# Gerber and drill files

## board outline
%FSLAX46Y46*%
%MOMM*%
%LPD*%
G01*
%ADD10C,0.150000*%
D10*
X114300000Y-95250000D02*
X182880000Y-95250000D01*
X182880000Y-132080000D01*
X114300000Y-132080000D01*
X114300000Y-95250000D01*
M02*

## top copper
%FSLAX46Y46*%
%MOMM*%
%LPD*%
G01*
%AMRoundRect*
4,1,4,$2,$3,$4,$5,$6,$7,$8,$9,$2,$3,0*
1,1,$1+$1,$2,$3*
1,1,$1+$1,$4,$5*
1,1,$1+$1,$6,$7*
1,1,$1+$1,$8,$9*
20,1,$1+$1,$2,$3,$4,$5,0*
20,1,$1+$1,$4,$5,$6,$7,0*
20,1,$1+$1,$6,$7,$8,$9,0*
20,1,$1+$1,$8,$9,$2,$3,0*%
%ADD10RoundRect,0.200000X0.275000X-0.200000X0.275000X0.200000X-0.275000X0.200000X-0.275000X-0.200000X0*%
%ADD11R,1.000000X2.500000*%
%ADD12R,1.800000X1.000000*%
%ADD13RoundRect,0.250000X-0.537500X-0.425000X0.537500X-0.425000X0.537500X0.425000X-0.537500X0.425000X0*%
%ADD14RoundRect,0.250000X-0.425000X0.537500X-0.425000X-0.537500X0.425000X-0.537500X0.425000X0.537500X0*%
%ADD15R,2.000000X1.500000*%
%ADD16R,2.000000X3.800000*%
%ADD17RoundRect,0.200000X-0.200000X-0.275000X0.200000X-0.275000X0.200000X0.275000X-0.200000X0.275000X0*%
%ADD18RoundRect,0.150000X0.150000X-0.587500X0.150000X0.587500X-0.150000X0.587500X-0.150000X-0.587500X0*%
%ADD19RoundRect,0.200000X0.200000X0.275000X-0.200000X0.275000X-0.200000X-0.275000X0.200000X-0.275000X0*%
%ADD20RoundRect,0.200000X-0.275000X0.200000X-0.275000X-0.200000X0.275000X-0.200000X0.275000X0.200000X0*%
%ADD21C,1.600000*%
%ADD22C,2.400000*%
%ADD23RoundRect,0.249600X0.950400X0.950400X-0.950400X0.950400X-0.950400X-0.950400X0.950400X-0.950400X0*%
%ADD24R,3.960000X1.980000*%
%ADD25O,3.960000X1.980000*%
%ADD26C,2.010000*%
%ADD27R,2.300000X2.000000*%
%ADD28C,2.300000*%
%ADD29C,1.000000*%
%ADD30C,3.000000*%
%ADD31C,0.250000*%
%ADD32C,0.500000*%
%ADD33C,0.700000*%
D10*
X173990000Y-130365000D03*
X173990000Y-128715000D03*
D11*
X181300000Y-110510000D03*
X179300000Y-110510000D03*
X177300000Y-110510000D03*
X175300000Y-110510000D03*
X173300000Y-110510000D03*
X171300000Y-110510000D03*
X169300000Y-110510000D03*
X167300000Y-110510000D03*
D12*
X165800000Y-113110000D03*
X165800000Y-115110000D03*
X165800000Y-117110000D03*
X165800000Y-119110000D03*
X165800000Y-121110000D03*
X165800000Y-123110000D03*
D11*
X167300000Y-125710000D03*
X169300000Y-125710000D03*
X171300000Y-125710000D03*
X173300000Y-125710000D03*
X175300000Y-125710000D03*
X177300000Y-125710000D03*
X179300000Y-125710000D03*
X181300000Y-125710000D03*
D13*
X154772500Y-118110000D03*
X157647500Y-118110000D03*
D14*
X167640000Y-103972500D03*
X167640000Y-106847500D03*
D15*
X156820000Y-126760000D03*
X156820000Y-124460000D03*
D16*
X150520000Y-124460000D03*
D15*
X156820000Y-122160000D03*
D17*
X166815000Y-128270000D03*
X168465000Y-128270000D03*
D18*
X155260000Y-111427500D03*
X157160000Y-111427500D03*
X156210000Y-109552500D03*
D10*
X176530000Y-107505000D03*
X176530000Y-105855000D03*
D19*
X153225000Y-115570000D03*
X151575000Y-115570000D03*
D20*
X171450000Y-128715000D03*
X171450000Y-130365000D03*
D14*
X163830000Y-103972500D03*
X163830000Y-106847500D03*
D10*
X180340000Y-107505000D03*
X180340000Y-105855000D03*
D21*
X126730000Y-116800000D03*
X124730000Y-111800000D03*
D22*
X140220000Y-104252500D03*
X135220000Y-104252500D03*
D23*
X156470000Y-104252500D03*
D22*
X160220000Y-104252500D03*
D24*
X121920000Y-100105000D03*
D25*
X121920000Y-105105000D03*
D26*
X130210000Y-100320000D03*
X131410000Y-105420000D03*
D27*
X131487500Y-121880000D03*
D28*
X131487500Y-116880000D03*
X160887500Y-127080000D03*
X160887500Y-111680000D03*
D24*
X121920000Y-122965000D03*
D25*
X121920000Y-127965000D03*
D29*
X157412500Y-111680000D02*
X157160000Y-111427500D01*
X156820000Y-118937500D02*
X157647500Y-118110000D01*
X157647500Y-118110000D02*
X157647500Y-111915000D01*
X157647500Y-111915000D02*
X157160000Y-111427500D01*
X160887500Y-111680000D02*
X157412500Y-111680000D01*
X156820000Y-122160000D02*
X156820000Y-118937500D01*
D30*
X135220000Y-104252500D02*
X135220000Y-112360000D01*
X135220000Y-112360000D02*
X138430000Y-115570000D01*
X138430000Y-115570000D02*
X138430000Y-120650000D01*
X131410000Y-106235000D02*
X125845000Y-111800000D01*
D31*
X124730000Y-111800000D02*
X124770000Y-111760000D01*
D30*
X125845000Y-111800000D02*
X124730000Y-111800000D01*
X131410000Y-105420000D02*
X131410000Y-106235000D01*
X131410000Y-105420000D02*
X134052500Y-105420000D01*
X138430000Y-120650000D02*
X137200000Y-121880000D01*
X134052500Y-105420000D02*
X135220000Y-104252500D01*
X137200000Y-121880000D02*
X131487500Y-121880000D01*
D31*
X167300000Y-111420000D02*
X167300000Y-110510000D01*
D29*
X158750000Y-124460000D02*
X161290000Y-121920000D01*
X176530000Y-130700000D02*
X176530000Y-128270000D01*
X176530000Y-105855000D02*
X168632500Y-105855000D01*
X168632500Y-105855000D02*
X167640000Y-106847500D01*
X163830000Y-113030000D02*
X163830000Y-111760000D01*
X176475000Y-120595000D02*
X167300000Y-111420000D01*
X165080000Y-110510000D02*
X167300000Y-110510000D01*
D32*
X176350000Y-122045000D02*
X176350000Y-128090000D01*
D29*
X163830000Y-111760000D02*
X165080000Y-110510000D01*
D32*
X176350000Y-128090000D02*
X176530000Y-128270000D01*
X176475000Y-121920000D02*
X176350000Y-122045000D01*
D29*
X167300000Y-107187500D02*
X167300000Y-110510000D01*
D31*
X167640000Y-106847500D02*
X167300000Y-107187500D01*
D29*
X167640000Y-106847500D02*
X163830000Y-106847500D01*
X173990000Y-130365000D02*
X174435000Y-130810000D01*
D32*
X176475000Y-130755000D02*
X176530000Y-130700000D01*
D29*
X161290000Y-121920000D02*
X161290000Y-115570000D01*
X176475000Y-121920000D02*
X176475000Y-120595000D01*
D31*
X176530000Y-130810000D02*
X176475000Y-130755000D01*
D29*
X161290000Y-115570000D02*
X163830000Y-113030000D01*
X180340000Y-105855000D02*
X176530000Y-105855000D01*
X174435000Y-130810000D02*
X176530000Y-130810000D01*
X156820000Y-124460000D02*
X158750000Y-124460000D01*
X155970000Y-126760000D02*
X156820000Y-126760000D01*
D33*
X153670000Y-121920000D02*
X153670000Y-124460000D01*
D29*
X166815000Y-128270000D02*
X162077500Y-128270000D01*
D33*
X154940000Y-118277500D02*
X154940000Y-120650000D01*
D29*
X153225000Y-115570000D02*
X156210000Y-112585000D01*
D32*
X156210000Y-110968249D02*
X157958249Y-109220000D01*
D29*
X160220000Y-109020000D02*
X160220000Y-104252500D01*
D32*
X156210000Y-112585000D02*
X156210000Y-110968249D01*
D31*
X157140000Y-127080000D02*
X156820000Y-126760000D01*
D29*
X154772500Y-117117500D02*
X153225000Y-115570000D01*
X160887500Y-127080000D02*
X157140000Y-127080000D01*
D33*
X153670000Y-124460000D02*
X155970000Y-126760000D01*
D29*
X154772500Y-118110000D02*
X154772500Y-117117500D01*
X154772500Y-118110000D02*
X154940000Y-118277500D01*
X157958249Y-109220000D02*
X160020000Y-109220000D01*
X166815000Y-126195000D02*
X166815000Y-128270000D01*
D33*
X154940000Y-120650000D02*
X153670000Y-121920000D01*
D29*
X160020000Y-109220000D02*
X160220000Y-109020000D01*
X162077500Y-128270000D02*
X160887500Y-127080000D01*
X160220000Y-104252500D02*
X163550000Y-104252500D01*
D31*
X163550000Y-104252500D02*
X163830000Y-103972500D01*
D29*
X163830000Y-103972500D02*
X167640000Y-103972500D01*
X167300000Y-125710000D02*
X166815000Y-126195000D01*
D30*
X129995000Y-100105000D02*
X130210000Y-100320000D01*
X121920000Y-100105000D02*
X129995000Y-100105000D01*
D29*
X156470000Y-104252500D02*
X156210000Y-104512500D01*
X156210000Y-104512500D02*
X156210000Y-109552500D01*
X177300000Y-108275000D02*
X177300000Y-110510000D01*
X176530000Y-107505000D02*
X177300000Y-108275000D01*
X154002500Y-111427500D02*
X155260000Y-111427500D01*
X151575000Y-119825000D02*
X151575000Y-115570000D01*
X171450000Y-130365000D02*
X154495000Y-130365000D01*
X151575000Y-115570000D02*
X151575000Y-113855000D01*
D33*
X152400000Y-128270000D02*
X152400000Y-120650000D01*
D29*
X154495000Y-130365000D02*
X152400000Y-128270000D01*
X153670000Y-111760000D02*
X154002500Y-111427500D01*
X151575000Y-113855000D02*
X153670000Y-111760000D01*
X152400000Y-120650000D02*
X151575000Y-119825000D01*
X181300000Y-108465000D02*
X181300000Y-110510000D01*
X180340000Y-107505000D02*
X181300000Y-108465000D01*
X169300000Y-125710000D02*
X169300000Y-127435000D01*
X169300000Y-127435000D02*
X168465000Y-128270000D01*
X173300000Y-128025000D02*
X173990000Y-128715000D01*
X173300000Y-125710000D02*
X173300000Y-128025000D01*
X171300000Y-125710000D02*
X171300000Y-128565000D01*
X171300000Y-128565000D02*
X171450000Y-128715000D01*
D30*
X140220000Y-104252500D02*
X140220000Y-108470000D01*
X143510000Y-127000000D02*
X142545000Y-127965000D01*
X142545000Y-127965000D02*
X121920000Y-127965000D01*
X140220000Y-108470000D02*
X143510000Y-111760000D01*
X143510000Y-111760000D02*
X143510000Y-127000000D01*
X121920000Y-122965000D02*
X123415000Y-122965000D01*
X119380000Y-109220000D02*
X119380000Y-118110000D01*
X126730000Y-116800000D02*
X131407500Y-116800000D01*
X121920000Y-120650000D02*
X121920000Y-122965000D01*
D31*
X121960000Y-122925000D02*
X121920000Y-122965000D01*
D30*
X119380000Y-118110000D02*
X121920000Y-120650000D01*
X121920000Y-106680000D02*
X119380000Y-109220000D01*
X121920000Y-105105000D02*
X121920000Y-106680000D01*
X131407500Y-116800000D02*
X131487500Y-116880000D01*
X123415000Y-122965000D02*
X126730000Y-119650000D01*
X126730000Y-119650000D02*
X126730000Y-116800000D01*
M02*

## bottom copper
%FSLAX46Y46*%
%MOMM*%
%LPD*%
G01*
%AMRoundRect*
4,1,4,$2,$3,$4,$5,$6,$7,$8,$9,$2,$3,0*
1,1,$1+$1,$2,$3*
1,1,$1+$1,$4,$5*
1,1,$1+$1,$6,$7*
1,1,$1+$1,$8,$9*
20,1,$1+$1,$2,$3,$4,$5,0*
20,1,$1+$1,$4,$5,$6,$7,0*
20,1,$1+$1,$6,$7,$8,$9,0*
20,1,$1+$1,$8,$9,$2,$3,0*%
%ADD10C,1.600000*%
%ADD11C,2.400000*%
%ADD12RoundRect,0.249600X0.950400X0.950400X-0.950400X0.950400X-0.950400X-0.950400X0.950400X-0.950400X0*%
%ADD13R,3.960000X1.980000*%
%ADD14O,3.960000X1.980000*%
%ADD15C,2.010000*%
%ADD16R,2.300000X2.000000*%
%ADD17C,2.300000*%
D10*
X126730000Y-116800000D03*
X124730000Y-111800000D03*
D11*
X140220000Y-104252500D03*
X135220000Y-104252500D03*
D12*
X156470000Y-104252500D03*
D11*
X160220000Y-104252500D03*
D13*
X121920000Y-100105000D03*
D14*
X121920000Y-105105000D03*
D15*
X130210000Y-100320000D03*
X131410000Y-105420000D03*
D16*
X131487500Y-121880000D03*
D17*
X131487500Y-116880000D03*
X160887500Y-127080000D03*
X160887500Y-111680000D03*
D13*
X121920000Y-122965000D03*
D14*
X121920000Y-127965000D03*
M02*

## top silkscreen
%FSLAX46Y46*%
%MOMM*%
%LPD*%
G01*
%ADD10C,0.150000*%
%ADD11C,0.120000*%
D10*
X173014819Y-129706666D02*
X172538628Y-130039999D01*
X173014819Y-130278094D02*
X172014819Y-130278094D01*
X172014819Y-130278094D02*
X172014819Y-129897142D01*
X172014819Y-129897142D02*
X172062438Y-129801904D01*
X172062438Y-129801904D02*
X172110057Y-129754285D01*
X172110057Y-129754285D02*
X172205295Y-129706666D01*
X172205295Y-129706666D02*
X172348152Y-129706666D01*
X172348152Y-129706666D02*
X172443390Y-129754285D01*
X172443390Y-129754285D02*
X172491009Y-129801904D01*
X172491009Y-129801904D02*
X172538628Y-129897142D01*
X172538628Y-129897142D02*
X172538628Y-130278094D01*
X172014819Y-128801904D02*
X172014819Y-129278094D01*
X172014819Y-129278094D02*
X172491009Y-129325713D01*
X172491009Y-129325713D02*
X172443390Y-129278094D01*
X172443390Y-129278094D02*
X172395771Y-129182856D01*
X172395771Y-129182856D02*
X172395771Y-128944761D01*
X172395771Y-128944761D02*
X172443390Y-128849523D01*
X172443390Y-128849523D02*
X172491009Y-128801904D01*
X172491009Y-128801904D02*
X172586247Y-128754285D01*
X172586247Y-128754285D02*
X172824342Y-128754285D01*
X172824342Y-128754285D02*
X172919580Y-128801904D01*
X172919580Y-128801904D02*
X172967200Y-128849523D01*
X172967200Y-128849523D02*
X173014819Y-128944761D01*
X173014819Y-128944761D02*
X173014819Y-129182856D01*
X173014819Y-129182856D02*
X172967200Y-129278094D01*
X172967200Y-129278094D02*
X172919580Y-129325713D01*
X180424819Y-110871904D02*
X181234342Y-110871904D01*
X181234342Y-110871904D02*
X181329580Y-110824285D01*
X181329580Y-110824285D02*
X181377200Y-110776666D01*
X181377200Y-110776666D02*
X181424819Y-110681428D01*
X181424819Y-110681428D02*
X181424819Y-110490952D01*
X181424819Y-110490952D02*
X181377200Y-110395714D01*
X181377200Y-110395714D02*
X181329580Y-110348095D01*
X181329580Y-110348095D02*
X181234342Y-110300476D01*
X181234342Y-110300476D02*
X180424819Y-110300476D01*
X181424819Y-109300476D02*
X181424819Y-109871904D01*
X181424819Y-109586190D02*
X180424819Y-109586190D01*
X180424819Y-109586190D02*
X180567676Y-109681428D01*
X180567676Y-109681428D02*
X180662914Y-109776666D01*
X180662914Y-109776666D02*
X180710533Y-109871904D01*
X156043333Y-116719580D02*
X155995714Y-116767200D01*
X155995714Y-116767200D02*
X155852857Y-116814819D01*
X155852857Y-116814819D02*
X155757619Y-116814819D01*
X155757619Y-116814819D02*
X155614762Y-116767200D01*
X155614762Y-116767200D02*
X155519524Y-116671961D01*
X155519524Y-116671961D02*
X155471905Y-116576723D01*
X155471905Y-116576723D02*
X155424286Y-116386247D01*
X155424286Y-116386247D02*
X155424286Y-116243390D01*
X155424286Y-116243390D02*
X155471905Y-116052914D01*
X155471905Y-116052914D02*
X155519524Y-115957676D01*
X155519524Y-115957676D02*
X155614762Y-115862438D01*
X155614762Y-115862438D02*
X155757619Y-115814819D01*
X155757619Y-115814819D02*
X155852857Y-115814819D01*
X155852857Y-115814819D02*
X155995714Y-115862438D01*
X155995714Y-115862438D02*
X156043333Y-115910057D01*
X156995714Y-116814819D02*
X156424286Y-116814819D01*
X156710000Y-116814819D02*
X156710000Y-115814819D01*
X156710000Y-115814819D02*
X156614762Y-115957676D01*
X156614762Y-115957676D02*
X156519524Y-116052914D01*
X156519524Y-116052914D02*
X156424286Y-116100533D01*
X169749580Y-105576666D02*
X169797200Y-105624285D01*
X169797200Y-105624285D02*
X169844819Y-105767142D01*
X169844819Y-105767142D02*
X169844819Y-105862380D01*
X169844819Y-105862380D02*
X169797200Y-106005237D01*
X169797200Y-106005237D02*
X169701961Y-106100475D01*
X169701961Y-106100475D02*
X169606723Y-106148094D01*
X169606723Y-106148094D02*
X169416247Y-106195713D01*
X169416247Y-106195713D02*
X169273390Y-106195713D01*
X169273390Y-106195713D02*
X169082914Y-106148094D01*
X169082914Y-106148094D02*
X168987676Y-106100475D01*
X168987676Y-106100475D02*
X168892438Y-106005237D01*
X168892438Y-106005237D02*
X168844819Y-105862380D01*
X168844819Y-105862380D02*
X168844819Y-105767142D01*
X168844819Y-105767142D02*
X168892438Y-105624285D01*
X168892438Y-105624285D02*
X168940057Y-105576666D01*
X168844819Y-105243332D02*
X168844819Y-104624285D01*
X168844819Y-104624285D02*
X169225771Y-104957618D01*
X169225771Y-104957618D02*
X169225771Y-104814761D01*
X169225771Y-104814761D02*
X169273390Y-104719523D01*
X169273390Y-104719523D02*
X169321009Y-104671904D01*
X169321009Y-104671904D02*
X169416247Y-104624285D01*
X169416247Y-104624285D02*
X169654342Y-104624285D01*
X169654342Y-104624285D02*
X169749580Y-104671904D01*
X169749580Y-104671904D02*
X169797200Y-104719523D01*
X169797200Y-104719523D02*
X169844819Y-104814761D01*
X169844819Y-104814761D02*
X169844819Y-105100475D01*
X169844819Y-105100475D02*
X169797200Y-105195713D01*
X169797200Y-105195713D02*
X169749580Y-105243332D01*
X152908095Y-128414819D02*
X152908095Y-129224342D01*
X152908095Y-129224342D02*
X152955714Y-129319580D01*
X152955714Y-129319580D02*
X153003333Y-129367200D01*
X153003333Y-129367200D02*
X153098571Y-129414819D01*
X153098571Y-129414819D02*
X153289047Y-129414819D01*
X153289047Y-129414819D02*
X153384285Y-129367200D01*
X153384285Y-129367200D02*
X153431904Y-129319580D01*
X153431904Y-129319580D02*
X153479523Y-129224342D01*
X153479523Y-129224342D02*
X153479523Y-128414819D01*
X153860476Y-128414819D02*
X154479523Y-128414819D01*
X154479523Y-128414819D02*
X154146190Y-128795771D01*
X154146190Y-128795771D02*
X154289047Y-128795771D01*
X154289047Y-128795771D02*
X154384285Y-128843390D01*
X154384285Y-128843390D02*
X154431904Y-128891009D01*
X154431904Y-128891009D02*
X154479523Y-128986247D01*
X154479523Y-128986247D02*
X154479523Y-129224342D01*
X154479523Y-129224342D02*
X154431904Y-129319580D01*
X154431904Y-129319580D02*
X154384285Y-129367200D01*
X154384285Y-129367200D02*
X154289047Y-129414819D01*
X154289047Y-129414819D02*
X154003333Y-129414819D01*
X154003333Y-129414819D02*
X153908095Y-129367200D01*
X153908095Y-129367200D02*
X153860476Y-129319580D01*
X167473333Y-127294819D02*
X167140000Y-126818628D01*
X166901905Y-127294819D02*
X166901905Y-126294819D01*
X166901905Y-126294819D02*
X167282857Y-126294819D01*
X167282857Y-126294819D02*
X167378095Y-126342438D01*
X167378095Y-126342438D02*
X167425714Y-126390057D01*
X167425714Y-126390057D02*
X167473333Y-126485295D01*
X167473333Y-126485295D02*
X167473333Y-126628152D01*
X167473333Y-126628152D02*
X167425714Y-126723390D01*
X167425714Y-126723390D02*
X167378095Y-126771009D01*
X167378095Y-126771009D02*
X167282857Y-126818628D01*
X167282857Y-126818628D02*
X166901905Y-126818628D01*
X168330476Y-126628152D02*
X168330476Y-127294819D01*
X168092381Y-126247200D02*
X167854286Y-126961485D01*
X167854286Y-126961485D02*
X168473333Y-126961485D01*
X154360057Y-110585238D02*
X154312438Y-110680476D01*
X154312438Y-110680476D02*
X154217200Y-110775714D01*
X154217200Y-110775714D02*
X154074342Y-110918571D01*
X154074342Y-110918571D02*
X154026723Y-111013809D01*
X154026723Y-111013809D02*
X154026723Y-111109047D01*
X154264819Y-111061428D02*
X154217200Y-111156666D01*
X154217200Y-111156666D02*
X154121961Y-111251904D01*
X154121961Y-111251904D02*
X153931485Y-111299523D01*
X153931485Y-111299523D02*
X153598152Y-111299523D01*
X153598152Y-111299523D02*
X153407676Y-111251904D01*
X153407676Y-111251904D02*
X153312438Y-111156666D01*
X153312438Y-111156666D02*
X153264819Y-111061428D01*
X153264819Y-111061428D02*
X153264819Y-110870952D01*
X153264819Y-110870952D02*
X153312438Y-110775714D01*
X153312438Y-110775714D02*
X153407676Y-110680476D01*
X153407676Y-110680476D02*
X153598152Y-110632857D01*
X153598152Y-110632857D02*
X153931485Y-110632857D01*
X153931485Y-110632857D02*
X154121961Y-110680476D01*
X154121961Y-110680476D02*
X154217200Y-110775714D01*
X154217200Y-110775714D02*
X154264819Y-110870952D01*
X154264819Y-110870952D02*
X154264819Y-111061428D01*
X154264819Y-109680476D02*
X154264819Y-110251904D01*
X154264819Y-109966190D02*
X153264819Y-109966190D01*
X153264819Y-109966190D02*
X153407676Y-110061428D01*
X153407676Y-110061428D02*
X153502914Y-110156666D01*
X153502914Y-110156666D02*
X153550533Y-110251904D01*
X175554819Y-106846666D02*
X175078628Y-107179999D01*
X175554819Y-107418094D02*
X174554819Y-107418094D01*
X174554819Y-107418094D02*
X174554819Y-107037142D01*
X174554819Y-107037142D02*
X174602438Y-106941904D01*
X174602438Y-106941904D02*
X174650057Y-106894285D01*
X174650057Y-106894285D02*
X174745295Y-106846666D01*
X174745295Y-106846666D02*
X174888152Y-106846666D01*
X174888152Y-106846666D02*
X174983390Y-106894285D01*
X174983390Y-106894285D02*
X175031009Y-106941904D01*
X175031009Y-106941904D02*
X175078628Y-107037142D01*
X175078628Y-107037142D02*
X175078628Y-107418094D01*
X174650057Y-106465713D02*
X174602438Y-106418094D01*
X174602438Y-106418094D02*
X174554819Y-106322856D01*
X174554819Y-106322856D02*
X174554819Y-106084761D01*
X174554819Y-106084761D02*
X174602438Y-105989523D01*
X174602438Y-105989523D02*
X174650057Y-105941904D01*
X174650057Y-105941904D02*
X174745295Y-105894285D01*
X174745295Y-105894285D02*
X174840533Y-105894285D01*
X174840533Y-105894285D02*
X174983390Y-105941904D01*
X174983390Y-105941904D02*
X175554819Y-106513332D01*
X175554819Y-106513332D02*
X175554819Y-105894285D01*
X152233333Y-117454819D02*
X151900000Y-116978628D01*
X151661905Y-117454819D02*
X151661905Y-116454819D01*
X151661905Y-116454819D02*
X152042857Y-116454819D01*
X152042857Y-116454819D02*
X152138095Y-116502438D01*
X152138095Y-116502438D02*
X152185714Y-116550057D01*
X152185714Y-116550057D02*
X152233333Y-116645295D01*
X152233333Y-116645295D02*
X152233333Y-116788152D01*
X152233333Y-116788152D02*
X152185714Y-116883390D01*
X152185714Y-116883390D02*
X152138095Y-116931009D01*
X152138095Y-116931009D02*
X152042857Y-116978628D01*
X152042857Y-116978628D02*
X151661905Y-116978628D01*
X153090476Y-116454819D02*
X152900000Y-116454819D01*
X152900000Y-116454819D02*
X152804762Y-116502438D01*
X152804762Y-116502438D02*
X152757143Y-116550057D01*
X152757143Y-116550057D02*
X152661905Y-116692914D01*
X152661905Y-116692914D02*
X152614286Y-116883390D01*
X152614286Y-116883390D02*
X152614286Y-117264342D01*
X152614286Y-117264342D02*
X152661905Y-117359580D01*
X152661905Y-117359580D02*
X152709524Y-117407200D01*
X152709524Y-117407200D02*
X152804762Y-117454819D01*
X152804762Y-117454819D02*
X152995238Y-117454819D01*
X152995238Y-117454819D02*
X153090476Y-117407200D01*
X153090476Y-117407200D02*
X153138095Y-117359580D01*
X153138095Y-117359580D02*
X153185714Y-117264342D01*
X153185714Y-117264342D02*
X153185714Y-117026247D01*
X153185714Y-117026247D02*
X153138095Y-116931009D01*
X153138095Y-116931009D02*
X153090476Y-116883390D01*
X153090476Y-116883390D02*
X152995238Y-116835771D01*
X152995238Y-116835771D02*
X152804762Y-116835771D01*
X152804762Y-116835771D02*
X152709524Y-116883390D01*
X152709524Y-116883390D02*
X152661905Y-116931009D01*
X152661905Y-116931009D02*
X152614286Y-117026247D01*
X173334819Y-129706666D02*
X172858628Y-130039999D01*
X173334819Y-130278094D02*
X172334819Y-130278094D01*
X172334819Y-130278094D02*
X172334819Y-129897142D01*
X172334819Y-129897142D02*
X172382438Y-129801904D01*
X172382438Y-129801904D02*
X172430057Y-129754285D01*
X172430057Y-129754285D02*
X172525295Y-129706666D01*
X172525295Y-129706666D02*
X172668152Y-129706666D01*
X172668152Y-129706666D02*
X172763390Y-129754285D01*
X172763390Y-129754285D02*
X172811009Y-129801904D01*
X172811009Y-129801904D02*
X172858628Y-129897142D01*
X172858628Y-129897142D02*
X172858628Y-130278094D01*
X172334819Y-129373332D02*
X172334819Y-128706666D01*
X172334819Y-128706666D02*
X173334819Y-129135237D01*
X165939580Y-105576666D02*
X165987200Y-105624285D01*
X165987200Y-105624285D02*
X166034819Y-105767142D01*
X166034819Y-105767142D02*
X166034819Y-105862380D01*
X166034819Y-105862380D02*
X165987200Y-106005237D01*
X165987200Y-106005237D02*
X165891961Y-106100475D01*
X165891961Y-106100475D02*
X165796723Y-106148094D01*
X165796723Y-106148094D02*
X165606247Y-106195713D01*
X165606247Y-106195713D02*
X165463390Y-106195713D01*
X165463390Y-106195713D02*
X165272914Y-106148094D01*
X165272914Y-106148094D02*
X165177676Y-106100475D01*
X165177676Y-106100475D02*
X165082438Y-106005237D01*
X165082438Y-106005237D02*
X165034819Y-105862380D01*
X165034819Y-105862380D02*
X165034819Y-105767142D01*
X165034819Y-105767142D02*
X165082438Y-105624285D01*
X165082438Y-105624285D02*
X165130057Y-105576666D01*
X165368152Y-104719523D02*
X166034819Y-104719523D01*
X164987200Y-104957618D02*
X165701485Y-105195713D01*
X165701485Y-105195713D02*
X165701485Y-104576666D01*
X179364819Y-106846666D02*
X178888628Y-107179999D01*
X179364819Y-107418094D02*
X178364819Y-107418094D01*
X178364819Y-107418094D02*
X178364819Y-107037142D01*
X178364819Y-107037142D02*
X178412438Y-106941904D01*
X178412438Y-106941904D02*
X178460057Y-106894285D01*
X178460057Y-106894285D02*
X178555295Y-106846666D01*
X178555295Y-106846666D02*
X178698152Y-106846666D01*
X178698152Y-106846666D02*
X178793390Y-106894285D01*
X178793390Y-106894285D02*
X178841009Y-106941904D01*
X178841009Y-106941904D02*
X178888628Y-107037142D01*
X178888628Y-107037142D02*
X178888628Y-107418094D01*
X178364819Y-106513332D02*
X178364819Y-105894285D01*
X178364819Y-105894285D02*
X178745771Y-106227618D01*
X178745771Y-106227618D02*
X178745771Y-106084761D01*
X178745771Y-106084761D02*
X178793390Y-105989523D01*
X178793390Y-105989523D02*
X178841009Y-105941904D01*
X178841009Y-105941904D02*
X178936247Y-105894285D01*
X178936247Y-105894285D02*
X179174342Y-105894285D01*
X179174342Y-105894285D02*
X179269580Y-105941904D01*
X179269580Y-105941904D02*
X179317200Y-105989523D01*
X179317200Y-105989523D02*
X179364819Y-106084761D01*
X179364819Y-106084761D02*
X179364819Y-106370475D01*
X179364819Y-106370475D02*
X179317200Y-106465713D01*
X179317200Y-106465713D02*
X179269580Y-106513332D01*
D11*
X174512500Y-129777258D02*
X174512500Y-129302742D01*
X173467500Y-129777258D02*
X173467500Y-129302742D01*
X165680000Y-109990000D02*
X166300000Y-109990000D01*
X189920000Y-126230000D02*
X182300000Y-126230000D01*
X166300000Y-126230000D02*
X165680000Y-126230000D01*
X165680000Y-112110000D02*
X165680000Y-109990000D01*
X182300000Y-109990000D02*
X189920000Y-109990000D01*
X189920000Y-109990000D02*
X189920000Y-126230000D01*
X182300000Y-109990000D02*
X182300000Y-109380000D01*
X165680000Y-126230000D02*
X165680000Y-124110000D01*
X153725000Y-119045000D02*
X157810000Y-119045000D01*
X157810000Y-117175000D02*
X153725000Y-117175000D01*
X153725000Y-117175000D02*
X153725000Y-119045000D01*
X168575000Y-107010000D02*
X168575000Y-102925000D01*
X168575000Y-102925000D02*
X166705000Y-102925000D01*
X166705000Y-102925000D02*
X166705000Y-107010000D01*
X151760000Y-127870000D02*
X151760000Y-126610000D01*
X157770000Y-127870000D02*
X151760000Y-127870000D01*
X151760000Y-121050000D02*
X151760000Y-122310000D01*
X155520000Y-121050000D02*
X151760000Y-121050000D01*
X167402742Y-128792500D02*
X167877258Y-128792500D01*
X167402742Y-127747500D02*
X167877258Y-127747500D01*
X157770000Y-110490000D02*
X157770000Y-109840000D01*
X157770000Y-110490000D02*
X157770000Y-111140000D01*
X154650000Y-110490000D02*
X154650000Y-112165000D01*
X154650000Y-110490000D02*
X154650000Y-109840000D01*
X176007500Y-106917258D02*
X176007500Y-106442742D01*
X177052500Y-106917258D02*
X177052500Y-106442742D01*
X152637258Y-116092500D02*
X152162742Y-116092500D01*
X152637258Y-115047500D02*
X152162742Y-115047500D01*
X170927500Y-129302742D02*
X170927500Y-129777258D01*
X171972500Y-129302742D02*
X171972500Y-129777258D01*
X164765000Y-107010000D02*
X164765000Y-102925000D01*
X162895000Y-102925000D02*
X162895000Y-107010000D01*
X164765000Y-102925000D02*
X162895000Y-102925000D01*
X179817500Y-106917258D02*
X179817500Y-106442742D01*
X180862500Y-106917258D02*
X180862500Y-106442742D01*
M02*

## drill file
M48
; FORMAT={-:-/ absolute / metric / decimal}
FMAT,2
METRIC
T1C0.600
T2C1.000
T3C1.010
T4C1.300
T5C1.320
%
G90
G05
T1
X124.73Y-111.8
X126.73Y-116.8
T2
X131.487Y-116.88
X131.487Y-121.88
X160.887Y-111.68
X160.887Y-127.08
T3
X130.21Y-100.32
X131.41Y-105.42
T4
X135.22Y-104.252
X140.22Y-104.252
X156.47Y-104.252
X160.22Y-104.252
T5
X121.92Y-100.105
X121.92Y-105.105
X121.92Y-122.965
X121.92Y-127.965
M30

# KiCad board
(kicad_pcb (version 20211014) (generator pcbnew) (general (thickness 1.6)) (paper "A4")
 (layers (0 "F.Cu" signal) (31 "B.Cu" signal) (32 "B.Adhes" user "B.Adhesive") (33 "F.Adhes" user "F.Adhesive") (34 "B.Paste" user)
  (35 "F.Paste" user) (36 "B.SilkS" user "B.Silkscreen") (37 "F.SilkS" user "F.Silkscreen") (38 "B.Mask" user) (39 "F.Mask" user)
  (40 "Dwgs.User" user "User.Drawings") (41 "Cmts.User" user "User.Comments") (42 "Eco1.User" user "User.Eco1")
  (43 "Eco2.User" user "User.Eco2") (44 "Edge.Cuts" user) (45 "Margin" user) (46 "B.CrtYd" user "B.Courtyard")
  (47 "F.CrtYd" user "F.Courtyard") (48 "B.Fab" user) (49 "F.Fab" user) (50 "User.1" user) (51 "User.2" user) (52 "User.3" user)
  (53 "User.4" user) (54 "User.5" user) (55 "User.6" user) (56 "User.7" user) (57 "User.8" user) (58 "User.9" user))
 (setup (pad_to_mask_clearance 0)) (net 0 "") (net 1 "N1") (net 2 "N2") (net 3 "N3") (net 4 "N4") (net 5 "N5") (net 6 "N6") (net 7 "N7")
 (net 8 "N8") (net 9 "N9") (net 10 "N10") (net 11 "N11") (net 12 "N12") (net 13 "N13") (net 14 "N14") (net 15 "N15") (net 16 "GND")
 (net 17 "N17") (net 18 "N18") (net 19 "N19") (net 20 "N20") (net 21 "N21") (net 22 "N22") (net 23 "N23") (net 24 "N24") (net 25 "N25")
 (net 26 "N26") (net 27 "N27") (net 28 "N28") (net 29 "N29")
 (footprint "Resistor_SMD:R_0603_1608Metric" (layer "F.Cu") (at 173.99 129.54 90)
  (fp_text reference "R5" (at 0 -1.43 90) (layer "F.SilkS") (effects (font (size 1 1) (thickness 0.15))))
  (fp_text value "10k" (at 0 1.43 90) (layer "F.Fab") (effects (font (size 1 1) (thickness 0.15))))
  (fp_line (start -0.237258 0.5225) (end 0.237258 0.5225) (layer "F.SilkS") (width 0.12))
  (fp_line (start -0.237258 -0.5225) (end 0.237258 -0.5225) (layer "F.SilkS") (width 0.12))
  (pad "1" smd roundrect (at -0.825 0 90) (size 0.8 0.95) (layers "F.Cu" "F.Paste" "F.Mask") (roundrect_rratio 0.25) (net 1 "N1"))
  (pad "2" smd roundrect (at 0.825 0 90) (size 0.8 0.95) (layers "F.Cu" "F.Paste" "F.Mask") (roundrect_rratio 0.25) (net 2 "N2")))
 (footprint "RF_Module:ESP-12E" (layer "F.Cu") (at 177.8 118.11 -90)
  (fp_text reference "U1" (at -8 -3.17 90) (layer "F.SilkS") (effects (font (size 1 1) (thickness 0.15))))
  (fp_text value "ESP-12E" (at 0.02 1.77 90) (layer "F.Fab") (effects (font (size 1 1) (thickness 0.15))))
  (fp_line (start -8.12 12.12) (end -8.12 11.5) (layer "F.SilkS") (width 0.12))
  (fp_line (start 8.12 -12.12) (end 8.12 -4.5) (layer "F.SilkS") (width 0.12))
  (fp_line (start 8.12 11.5) (end 8.12 12.12) (layer "F.SilkS") (width 0.12))
  (fp_line (start -6 12.12) (end -8.12 12.12) (layer "F.SilkS") (width 0.12))
  (fp_line (start -8.12 -4.5) (end -8.12 -12.12) (layer "F.SilkS") (width 0.12))
  (fp_line (start -8.12 -12.12) (end 8.12 -12.12) (layer "F.SilkS") (width 0.12))
  (fp_line (start -8.12 -4.5) (end -8.73 -4.5) (layer "F.SilkS") (width 0.12))
  (fp_line (start 8.12 12.12) (end 6 12.12) (layer "F.SilkS") (width 0.12))
  (pad "1" smd rect (at -7.6 -3.5 270) (size 2.5 1) (layers "F.Cu" "F.Paste" "F.Mask") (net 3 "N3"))
  (pad "2" smd rect (at -7.6 -1.5 270) (size 2.5 1) (layers "F.Cu" "F.Paste" "F.Mask") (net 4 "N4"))
  (pad "3" smd rect (at -7.6 0.5 270) (size 2.5 1) (layers "F.Cu" "F.Paste" "F.Mask") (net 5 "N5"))
  (pad "4" smd rect (at -7.6 2.5 270) (size 2.5 1) (layers "F.Cu" "F.Paste" "F.Mask") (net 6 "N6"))
  (pad "5" smd rect (at -7.6 4.5 270) (size 2.5 1) (layers "F.Cu" "F.Paste" "F.Mask") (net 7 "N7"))
  (pad "6" smd rect (at -7.6 6.5 270) (size 2.5 1) (layers "F.Cu" "F.Paste" "F.Mask") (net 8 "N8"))
  (pad "7" smd rect (at -7.6 8.5 270) (size 2.5 1) (layers "F.Cu" "F.Paste" "F.Mask") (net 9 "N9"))
  (pad "8" smd rect (at -7.6 10.5 270) (size 2.5 1) (layers "F.Cu" "F.Paste" "F.Mask") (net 1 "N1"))
  (pad "9" smd rect (at -5 12 270) (size 1 1.8) (layers "F.Cu" "F.Paste" "F.Mask") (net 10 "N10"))
  (pad "10" smd rect (at -3 12 270) (size 1 1.8) (layers "F.Cu" "F.Paste" "F.Mask") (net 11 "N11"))
  (pad "11" smd rect (at -1 12 270) (size 1 1.8) (layers "F.Cu" "F.Paste" "F.Mask") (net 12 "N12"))
  (pad "12" smd rect (at 1 12 270) (size 1 1.8) (layers "F.Cu" "F.Paste" "F.Mask") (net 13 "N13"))
  (pad "13" smd rect (at 3 12 270) (size 1 1.8) (layers "F.Cu" "F.Paste" "F.Mask") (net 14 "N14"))
  (pad "14" smd rect (at 5 12 270) (size 1 1.8) (layers "F.Cu" "F.Paste" "F.Mask") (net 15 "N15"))
  (pad "15" smd rect (at 7.6 10.5 270) (size 2.5 1) (layers "F.Cu" "F.Paste" "F.Mask") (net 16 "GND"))
  (pad "16" smd rect (at 7.6 8.5 270) (size 2.5 1) (layers "F.Cu" "F.Paste" "F.Mask") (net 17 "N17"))
  (pad "17" smd rect (at 7.6 6.5 270) (size 2.5 1) (layers "F.Cu" "F.Paste" "F.Mask") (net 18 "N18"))
  (pad "18" smd rect (at 7.6 4.5 270) (size 2.5 1) (layers "F.Cu" "F.Paste" "F.Mask") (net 2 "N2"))
  (pad "19" smd rect (at 7.6 2.5 270) (size 2.5 1) (layers "F.Cu" "F.Paste" "F.Mask") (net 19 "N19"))
  (pad "20" smd rect (at 7.6 0.5 270) (size 2.5 1) (layers "F.Cu" "F.Paste" "F.Mask") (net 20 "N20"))
  (pad "21" smd rect (at 7.6 -1.5 270) (size 2.5 1) (layers "F.Cu" "F.Paste" "F.Mask") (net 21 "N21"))
  (pad "22" smd rect (at 7.6 -3.5 270) (size 2.5 1) (layers "F.Cu" "F.Paste" "F.Mask") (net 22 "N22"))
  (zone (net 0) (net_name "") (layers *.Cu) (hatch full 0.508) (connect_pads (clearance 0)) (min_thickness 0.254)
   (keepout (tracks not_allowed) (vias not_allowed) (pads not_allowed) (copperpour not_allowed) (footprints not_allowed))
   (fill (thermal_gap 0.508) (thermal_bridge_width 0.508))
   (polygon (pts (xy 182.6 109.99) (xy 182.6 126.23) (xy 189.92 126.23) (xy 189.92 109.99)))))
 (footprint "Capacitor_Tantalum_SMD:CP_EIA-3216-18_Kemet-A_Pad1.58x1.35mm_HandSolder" (layer "F.Cu") (at 156.21 118.11)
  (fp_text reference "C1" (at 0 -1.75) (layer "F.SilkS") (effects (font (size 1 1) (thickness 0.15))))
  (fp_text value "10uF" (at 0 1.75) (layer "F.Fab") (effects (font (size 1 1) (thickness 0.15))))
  (fp_line (start -2.485 0.935) (end 1.6 0.935) (layer "F.SilkS") (width 0.12))
  (fp_line (start 1.6 -0.935) (end -2.485 -0.935) (layer "F.SilkS") (width 0.12))
  (fp_line (start -2.485 -0.935) (end -2.485 0.935) (layer "F.SilkS") (width 0.12))
  (pad "1" smd roundrect (at -1.4375 0) (size 1.575 1.35) (layers "F.Cu" "F.Paste" "F.Mask") (roundrect_rratio 0.1851851852) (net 16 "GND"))
  (pad "2" smd roundrect (at 1.4375 0) (size 1.575 1.35) (layers "F.Cu" "F.Paste" "F.Mask") (roundrect_rratio 0.1851851852) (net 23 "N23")))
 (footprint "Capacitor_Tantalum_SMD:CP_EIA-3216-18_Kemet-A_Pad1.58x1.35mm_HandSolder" (layer "F.Cu") (at 167.64 105.41 -90)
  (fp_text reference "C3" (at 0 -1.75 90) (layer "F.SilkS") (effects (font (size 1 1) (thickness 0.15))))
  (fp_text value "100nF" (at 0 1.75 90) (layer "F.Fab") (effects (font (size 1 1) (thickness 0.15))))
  (fp_line (start 1.6 -0.935) (end -2.485 -0.935) (layer "F.SilkS") (width 0.12))
  (fp_line (start -2.485 -0.935) (end -2.485 0.935) (layer "F.SilkS") (width 0.12))
  (fp_line (start -2.485 0.935) (end 1.6 0.935) (layer "F.SilkS") (width 0.12))
  (pad "1" smd roundrect (at -1.4375 0 270) (size 1.575 1.35) (layers "F.Cu" "F.Paste" "F.Mask") (roundrect_rratio 0.1851851852)
   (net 16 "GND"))
  (pad "2" smd roundrect (at 1.4375 0 270) (size 1.575 1.35) (layers "F.Cu" "F.Paste" "F.Mask") (roundrect_rratio 0.1851851852) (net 1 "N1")))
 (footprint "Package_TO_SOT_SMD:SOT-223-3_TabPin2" (layer "F.Cu") (at 153.67 124.46 180)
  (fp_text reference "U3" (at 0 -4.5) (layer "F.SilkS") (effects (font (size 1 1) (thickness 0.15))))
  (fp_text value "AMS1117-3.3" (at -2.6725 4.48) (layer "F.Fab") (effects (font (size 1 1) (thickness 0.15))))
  (fp_line (start 1.91 -3.41) (end 1.91 -2.15) (layer "F.SilkS") (width 0.12))
  (fp_line (start -4.1 -3.41) (end 1.91 -3.41) (layer "F.SilkS") (width 0.12))
  (fp_line (start 1.91 3.41) (end 1.91 2.15) (layer "F.SilkS") (width 0.12))
  (fp_line (start -1.85 3.41) (end 1.91 3.41) (layer "F.SilkS") (width 0.12))
  (pad "1" smd rect (at -3.15 -2.3 180) (size 2 1.5) (layers "F.Cu" "F.Paste" "F.Mask") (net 16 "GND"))
  (pad "2" smd rect (at -3.15 0 180) (size 2 1.5) (layers "F.Cu" "F.Paste" "F.Mask") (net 1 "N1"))
  (pad "2" smd rect (at 3.15 0 180) (size 2 3.8) (layers "F.Cu" "F.Paste" "F.Mask") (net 1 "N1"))
  (pad "3" smd rect (at -3.15 2.3 180) (size 2 1.5) (layers "F.Cu" "F.Paste" "F.Mask") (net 23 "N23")))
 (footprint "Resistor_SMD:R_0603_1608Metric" (layer "F.Cu") (at 167.64 128.27)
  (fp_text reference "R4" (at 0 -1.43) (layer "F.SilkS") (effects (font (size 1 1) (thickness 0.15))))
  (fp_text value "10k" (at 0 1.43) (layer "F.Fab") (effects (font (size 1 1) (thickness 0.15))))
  (fp_line (start -0.237258 0.5225) (end 0.237258 0.5225) (layer "F.SilkS") (width 0.12))
  (fp_line (start -0.237258 -0.5225) (end 0.237258 -0.5225) (layer "F.SilkS") (width 0.12))
  (pad "1" smd roundrect (at -0.825 0) (size 0.8 0.95) (layers "F.Cu" "F.Paste" "F.Mask") (roundrect_rratio 0.25) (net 16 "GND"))
  (pad "2" smd roundrect (at 0.825 0) (size 0.8 0.95) (layers "F.Cu" "F.Paste" "F.Mask") (roundrect_rratio 0.25) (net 17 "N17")))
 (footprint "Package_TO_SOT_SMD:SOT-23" (layer "F.Cu") (at 156.21 110.49 90)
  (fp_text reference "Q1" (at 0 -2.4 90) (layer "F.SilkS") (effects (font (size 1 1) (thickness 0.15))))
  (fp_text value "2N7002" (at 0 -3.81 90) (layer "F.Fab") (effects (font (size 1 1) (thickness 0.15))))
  (fp_line (start 0 1.56) (end 0.65 1.56) (layer "F.SilkS") (width 0.12))
  (fp_line (start 0 1.56) (end -0.65 1.56) (layer "F.SilkS") (width 0.12))
  (fp_line (start 0 -1.56) (end -1.675 -1.56) (layer "F.SilkS") (width 0.12))
  (fp_line (start 0 -1.56) (end 0.65 -1.56) (layer "F.SilkS") (width 0.12))
  (pad "1" smd roundrect (at -0.9375 -0.95 90) (size 1.475 0.6) (layers "F.Cu" "F.Paste" "F.Mask") (roundrect_rratio 0.25) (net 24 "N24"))
  (pad "2" smd roundrect (at -0.9375 0.95 90) (size 1.475 0.6) (layers "F.Cu" "F.Paste" "F.Mask") (roundrect_rratio 0.25) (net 23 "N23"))
  (pad "3" smd roundrect (at 0.9375 0 90) (size 1.475 0.6) (layers "F.Cu" "F.Paste" "F.Mask") (roundrect_rratio 0.25) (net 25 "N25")))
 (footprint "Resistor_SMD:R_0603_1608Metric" (layer "F.Cu") (at 176.53 106.68 90)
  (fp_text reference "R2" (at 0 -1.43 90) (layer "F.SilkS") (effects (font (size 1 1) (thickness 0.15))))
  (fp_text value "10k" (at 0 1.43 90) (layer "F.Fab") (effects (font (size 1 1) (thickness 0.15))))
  (fp_line (start -0.237258 -0.5225) (end 0.237258 -0.5225) (layer "F.SilkS") (width 0.12))
  (fp_line (start -0.237258 0.5225) (end 0.237258 0.5225) (layer "F.SilkS") (width 0.12))
  (pad "1" smd roundrect (at -0.825 0 90) (size 0.8 0.95) (layers "F.Cu" "F.Paste" "F.Mask") (roundrect_rratio 0.25) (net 5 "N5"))
  (pad "2" smd roundrect (at 0.825 0 90) (size 0.8 0.95) (layers "F.Cu" "F.Paste" "F.Mask") (roundrect_rratio 0.25) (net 1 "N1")))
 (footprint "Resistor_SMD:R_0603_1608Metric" (layer "F.Cu") (at 152.4 115.57 180)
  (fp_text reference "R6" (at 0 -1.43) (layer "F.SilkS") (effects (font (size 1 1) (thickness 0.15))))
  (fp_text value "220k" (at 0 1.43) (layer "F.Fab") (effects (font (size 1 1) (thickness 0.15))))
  (fp_line (start -0.237258 -0.5225) (end 0.237258 -0.5225) (layer "F.SilkS") (width 0.12))
  (fp_line (start -0.237258 0.5225) (end 0.237258 0.5225) (layer "F.SilkS") (width 0.12))
  (pad "1" smd roundrect (at -0.825 0 180) (size 0.8 0.95) (layers "F.Cu" "F.Paste" "F.Mask") (roundrect_rratio 0.25) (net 16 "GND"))
  (pad "2" smd roundrect (at 0.825 0 180) (size 0.8 0.95) (layers "F.Cu" "F.Paste" "F.Mask") (roundrect_rratio 0.25) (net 24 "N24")))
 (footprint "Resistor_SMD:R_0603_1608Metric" (layer "F.Cu") (at 171.45 129.54 -90)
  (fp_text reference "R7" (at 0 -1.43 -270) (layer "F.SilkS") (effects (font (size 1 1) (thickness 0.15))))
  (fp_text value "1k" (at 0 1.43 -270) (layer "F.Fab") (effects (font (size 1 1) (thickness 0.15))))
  (fp_line (start -0.237258 0.5225) (end 0.237258 0.5225) (layer "F.SilkS") (width 0.12))
  (fp_line (start -0.237258 -0.5225) (end 0.237258 -0.5225) (layer "F.SilkS") (width 0.12))
  (pad "1" smd roundrect (at -0.825 0 270) (size 0.8 0.95) (layers "F.Cu" "F.Paste" "F.Mask") (roundrect_rratio 0.25) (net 18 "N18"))
  (pad "2" smd roundrect (at 0.825 0 270) (size 0.8 0.95) (layers "F.Cu" "F.Paste" "F.Mask") (roundrect_rratio 0.25) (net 24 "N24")))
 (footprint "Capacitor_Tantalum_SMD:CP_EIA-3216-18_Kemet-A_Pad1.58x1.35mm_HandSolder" (layer "F.Cu") (at 163.83 105.41 -90)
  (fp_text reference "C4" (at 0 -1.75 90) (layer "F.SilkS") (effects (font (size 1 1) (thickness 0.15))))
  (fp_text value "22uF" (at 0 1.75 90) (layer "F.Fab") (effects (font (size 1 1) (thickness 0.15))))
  (fp_line (start 1.6 -0.935) (end -2.485 -0.935) (layer "F.SilkS") (width 0.12))
  (fp_line (start -2.485 0.935) (end 1.6 0.935) (layer "F.SilkS") (width 0.12))
  (fp_line (start -2.485 -0.935) (end -2.485 0.935) (layer "F.SilkS") (width 0.12))
  (pad "1" smd roundrect (at -1.4375 0 270) (size 1.575 1.35) (layers "F.Cu" "F.Paste" "F.Mask") (roundrect_rratio 0.1851851852)
   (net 16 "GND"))
  (pad "2" smd roundrect (at 1.4375 0 270) (size 1.575 1.35) (layers "F.Cu" "F.Paste" "F.Mask") (roundrect_rratio 0.1851851852) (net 1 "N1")))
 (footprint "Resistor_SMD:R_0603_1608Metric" (layer "F.Cu") (at 180.34 106.68 90)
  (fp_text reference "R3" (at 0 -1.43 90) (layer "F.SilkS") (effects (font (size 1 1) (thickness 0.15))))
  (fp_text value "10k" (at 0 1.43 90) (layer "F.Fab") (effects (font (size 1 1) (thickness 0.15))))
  (fp_line (start -0.237258 -0.5225) (end 0.237258 -0.5225) (layer "F.SilkS") (width 0.12))
  (fp_line (start -0.237258 0.5225) (end 0.237258 0.5225) (layer "F.SilkS") (width 0.12))
  (pad "1" smd roundrect (at -0.825 0 90) (size 0.8 0.95) (layers "F.Cu" "F.Paste" "F.Mask") (roundrect_rratio 0.25) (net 3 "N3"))
  (pad "2" smd roundrect (at 0.825 0 90) (size 0.8 0.95) (layers "F.Cu" "F.Paste" "F.Mask") (roundrect_rratio 0.25) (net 1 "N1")))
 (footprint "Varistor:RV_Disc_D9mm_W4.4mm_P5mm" (layer "B.Cu") (at 126.73 116.8 90)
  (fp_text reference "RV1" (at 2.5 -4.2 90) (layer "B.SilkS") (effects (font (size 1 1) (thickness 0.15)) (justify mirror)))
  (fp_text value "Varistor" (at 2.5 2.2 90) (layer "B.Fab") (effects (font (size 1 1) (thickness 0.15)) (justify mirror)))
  (pad "1" thru_hole circle (at 0 0 90) (size 1.6 1.6) (drill 0.6) (layers *.Cu *.Mask) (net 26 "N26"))
  (pad "2" thru_hole circle (at 5 -2 90) (size 1.6 1.6) (drill 0.6) (layers *.Cu *.Mask) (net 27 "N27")))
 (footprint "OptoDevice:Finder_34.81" (layer "B.Cu") (at 156.47 104.2525 180)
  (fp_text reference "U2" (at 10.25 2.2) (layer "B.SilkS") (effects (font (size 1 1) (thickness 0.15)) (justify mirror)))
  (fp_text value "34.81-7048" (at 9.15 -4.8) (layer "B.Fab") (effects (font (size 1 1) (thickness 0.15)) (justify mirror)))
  (pad "11" thru_hole circle (at 16.25 0 180) (size 2.4 2.4) (drill 1.3) (layers *.Cu *.Mask) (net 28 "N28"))
  (pad "14" thru_hole circle (at 21.25 0 180) (size 2.4 2.4) (drill 1.3) (layers *.Cu *.Mask) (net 27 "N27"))
  (pad "A1" thru_hole roundrect (at 0 0 180) (size 2.4 2.4) (drill 1.3) (layers *.Cu *.Mask) (roundrect_rratio 0.104) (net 25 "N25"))
  (pad "A2" thru_hole circle (at -3.75 0 180) (size 2.4 2.4) (drill 1.3) (layers *.Cu *.Mask) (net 16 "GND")))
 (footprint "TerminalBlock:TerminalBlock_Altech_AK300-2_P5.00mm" (layer "B.Cu") (at 121.92 100.105 -90)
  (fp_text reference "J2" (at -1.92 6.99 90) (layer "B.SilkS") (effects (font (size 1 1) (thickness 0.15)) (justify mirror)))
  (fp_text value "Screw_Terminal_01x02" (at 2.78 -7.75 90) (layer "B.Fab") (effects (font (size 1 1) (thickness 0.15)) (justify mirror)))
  (pad "1" thru_hole rect (at 0 0 270) (size 1.98 3.96) (drill 1.32) (layers *.Cu *.Mask) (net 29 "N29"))
  (pad "2" thru_hole oval (at 5 0 270) (size 1.98 3.96) (drill 1.32) (layers *.Cu *.Mask) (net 26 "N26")))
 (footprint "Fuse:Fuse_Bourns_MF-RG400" (layer "B.Cu") (at 130.21 100.32 -90)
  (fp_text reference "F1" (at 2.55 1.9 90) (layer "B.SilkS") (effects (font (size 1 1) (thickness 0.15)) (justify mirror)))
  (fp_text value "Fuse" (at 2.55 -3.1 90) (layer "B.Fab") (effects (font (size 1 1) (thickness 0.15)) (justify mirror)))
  (pad "1" thru_hole circle (at 0 0 270) (size 2.01 2.01) (drill 1.01) (layers *.Cu *.Mask) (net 29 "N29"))
  (pad "2" thru_hole circle (at 5.1 -1.2 270) (size 2.01 2.01) (drill 1.01) (layers *.Cu *.Mask) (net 27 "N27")))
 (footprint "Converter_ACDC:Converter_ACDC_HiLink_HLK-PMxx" (layer "B.Cu") (at 131.4875 121.88)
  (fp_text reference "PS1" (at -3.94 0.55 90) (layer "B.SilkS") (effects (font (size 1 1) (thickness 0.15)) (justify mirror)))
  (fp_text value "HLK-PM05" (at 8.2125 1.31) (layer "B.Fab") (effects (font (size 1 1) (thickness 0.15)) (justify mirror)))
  (pad "1" thru_hole rect (at 0 0) (size 2.3 2) (drill 1) (layers *.Cu *.Mask) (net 27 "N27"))
  (pad "2" thru_hole circle (at 0 -5) (size 2.3 2.3) (drill 1) (layers *.Cu *.Mask) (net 26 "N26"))
  (pad "3" thru_hole circle (at 29.4 5.2) (size 2.3 2.3) (drill 1) (layers *.Cu *.Mask) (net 16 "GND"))
  (pad "4" thru_hole circle (at 29.4 -10.2) (size 2.3 2.3) (drill 1) (layers *.Cu *.Mask) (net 23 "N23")))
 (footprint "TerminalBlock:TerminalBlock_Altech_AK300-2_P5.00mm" (layer "B.Cu") (at 121.92 122.965 -90)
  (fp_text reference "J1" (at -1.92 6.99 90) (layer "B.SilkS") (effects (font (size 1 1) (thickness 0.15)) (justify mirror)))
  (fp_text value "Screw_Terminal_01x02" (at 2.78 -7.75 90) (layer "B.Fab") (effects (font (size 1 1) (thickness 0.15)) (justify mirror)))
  (pad "1" thru_hole rect (at 0 0 270) (size 1.98 3.96) (drill 1.32) (layers *.Cu *.Mask) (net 26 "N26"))
  (pad "2" thru_hole oval (at 5 0 270) (size 1.98 3.96) (drill 1.32) (layers *.Cu *.Mask) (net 28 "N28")))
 (gr_rect (start 114.3 95.25) (end 182.88 132.08) (layer "Edge.Cuts") (width 0.15) (fill none))
 (segment (start 157.4125 111.68) (end 157.16 111.4275) (width 1) (layer "F.Cu") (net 23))
 (segment (start 156.82 118.9375) (end 157.6475 118.11) (width 1) (layer "F.Cu") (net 23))
 (segment (start 157.6475 118.11) (end 157.6475 111.915) (width 1) (layer "F.Cu") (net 23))
 (segment (start 157.6475 111.915) (end 157.16 111.4275) (width 1) (layer "F.Cu") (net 23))
 (segment (start 160.8875 111.68) (end 157.4125 111.68) (width 1) (layer "F.Cu") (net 23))
 (segment (start 156.82 122.16) (end 156.82 118.9375) (width 1) (layer "F.Cu") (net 23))
 (segment (start 135.22 104.2525) (end 135.22 112.36) (width 3) (layer "F.Cu") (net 27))
 (segment (start 135.22 112.36) (end 138.43 115.57) (width 3) (layer "F.Cu") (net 27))
 (segment (start 138.43 115.57) (end 138.43 120.65) (width 3) (layer "F.Cu") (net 27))
 (segment (start 131.41 106.235) (end 125.845 111.8) (width 3) (layer "F.Cu") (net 27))
 (segment (start 124.73 111.8) (end 124.77 111.76) (width 0.25) (layer "F.Cu") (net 27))
 (segment (start 125.845 111.8) (end 124.73 111.8) (width 3) (layer "F.Cu") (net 27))
 (segment (start 131.41 105.42) (end 131.41 106.235) (width 3) (layer "F.Cu") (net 27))
 (segment (start 131.41 105.42) (end 134.0525 105.42) (width 3) (layer "F.Cu") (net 27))
 (segment (start 138.43 120.65) (end 137.2 121.88) (width 3) (layer "F.Cu") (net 27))
 (segment (start 134.0525 105.42) (end 135.22 104.2525) (width 3) (layer "F.Cu") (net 27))
 (segment (start 137.2 121.88) (end 131.4875 121.88) (width 3) (layer "F.Cu") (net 27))
 (segment (start 167.3 111.42) (end 167.3 110.51) (width 0.25) (layer "F.Cu") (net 1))
 (segment (start 158.75 124.46) (end 161.29 121.92) (width 1) (layer "F.Cu") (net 1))
 (segment (start 176.53 130.7) (end 176.53 128.27) (width 1) (layer "F.Cu") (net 1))
 (segment (start 176.53 105.855) (end 168.6325 105.855) (width 1) (layer "F.Cu") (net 1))
 (segment (start 168.6325 105.855) (end 167.64 106.8475) (width 1) (layer "F.Cu") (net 1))
 (segment (start 163.83 113.03) (end 163.83 111.76) (width 1) (layer "F.Cu") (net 1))
 (segment (start 176.475 120.595) (end 167.3 111.42) (width 1) (layer "F.Cu") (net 1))
 (segment (start 165.08 110.51) (end 167.3 110.51) (width 1) (layer "F.Cu") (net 1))
 (segment (start 176.35 122.045) (end 176.35 128.09) (width 0.5) (layer "F.Cu") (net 1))
 (segment (start 163.83 111.76) (end 165.08 110.51) (width 1) (layer "F.Cu") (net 1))
 (segment (start 176.35 128.09) (end 176.53 128.27) (width 0.5) (layer "F.Cu") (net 1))
 (segment (start 176.475 121.92) (end 176.35 122.045) (width 0.5) (layer "F.Cu") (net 1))
 (segment (start 167.3 107.1875) (end 167.3 110.51) (width 1) (layer "F.Cu") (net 1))
 (segment (start 167.64 106.8475) (end 167.3 107.1875) (width 0.25) (layer "F.Cu") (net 1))
 (segment (start 167.64 106.8475) (end 163.83 106.8475) (width 1) (layer "F.Cu") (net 1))
 (segment (start 173.99 130.365) (end 174.435 130.81) (width 1) (layer "F.Cu") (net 1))
 (segment (start 176.475 130.755) (end 176.53 130.7) (width 0.5) (layer "F.Cu") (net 1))
 (segment (start 161.29 121.92) (end 161.29 115.57) (width 1) (layer "F.Cu") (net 1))
 (segment (start 176.475 121.92) (end 176.475 120.595) (width 1) (layer "F.Cu") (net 1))
 (segment (start 176.53 130.81) (end 176.475 130.755) (width 0.25) (layer "F.Cu") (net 1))
 (segment (start 161.29 115.57) (end 163.83 113.03) (width 1) (layer "F.Cu") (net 1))
 (segment (start 180.34 105.855) (end 176.53 105.855) (width 1) (layer "F.Cu") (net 1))
 (segment (start 174.435 130.81) (end 176.53 130.81) (width 1) (layer "F.Cu") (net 1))
 (segment (start 156.82 124.46) (end 158.75 124.46) (width 1) (layer "F.Cu") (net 1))
 (segment (start 155.97 126.76) (end 156.82 126.76) (width 1) (layer "F.Cu") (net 16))
 (segment (start 153.67 121.92) (end 153.67 124.46) (width 0.7) (layer "F.Cu") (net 16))
 (segment (start 166.815 128.27) (end 162.0775 128.27) (width 1) (layer "F.Cu") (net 16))
 (segment (start 154.94 118.2775) (end 154.94 120.65) (width 0.7) (layer "F.Cu") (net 16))
 (segment (start 153.225 115.57) (end 156.21 112.585) (width 1) (layer "F.Cu") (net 16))
 (segment (start 156.21 110.968249) (end 157.958249 109.22) (width 0.5) (layer "F.Cu") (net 16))
 (segment (start 160.22 109.02) (end 160.22 104.2525) (width 1) (layer "F.Cu") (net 16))
 (segment (start 156.21 112.585) (end 156.21 110.968249) (width 0.5) (layer "F.Cu") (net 16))
 (segment (start 157.14 127.08) (end 156.82 126.76) (width 0.25) (layer "F.Cu") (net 16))
 (segment (start 154.7725 117.1175) (end 153.225 115.57) (width 1) (layer "F.Cu") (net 16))
 (segment (start 160.8875 127.08) (end 157.14 127.08) (width 1) (layer "F.Cu") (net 16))
 (segment (start 153.67 124.46) (end 155.97 126.76) (width 0.7) (layer "F.Cu") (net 16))
 (segment (start 154.7725 118.11) (end 154.7725 117.1175) (width 1) (layer "F.Cu") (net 16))
 (segment (start 154.7725 118.11) (end 154.94 118.2775) (width 1) (layer "F.Cu") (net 16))
 (segment (start 157.958249 109.22) (end 160.02 109.22) (width 1) (layer "F.Cu") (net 16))
 (segment (start 166.815 126.195) (end 166.815 128.27) (width 1) (layer "F.Cu") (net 16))
 (segment (start 154.94 120.65) (end 153.67 121.92) (width 0.7) (layer "F.Cu") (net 16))
 (segment (start 160.02 109.22) (end 160.22 109.02) (width 1) (layer "F.Cu") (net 16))
 (segment (start 162.0775 128.27) (end 160.8875 127.08) (width 1) (layer "F.Cu") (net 16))
 (segment (start 160.22 104.2525) (end 163.55 104.2525) (width 1) (layer "F.Cu") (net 16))
 (segment (start 163.55 104.2525) (end 163.83 103.9725) (width 0.25) (layer "F.Cu") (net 16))
 (segment (start 163.83 103.9725) (end 167.64 103.9725) (width 1) (layer "F.Cu") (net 16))
 (segment (start 167.3 125.71) (end 166.815 126.195) (width 1) (layer "F.Cu") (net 16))
 (segment (start 129.995 100.105) (end 130.21 100.32) (width 3) (layer "F.Cu") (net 29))
 (segment (start 121.92 100.105) (end 129.995 100.105) (width 3) (layer "F.Cu") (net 29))
 (segment (start 156.47 104.2525) (end 156.21 104.5125) (width 1) (layer "F.Cu") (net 25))
 (segment (start 156.21 104.5125) (end 156.21 109.5525) (width 1) (layer "F.Cu") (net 25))
 (segment (start 177.3 108.275) (end 177.3 110.51) (width 1) (layer "F.Cu") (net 5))
 (segment (start 176.53 107.505) (end 177.3 108.275) (width 1) (layer "F.Cu") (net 5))
 (segment (start 154.0025 111.4275) (end 155.26 111.4275) (width 1) (layer "F.Cu") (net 24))
 (segment (start 151.575 119.825) (end 151.575 115.57) (width 1) (layer "F.Cu") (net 24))
 (segment (start 171.45 130.365) (end 154.495 130.365) (width 1) (layer "F.Cu") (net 24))
 (segment (start 151.575 115.57) (end 151.575 113.855) (width 1) (layer "F.Cu") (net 24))
 (segment (start 152.4 128.27) (end 152.4 120.65) (width 0.7) (layer "F.Cu") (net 24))
 (segment (start 154.495 130.365) (end 152.4 128.27) (width 1) (layer "F.Cu") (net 24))
 (segment (start 153.67 111.76) (end 154.0025 111.4275) (width 1) (layer "F.Cu") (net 24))
 (segment (start 151.575 113.855) (end 153.67 111.76) (width 1) (layer "F.Cu") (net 24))
 (segment (start 152.4 120.65) (end 151.575 119.825) (width 1) (layer "F.Cu") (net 24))
 (segment (start 181.3 108.465) (end 181.3 110.51) (width 1) (layer "F.Cu") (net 3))
 (segment (start 180.34 107.505) (end 181.3 108.465) (width 1) (layer "F.Cu") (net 3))
 (segment (start 169.3 125.71) (end 169.3 127.435) (width 1) (layer "F.Cu") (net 17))
 (segment (start 169.3 127.435) (end 168.465 128.27) (width 1) (layer "F.Cu") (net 17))
 (segment (start 173.3 128.025) (end 173.99 128.715) (width 1) (layer "F.Cu") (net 2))
 (segment (start 173.3 125.71) (end 173.3 128.025) (width 1) (layer "F.Cu") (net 2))
 (segment (start 171.3 125.71) (end 171.3 128.565) (width 1) (layer "F.Cu") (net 18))
 (segment (start 171.3 128.565) (end 171.45 128.715) (width 1) (layer "F.Cu") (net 18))
 (segment (start 140.22 104.2525) (end 140.22 108.47) (width 3) (layer "F.Cu") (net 28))
 (segment (start 143.51 127) (end 142.545 127.965) (width 3) (layer "F.Cu") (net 28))
 (segment (start 142.545 127.965) (end 121.92 127.965) (width 3) (layer "F.Cu") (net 28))
 (segment (start 140.22 108.47) (end 143.51 111.76) (width 3) (layer "F.Cu") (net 28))
 (segment (start 143.51 111.76) (end 143.51 127) (width 3) (layer "F.Cu") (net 28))
 (segment (start 121.92 122.965) (end 123.415 122.965) (width 3) (layer "F.Cu") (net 26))
 (segment (start 119.38 109.22) (end 119.38 118.11) (width 3) (layer "F.Cu") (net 26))
 (segment (start 126.73 116.8) (end 131.4075 116.8) (width 3) (layer "F.Cu") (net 26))
 (segment (start 121.92 120.65) (end 121.92 122.965) (width 3) (layer "F.Cu") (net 26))
 (segment (start 121.96 122.925) (end 121.92 122.965) (width 0.25) (layer "F.Cu") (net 26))
 (segment (start 119.38 118.11) (end 121.92 120.65) (width 3) (layer "F.Cu") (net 26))
 (segment (start 121.92 106.68) (end 119.38 109.22) (width 3) (layer "F.Cu") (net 26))
 (segment (start 121.92 105.105) (end 121.92 106.68) (width 3) (layer "F.Cu") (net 26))
 (segment (start 131.4075 116.8) (end 131.4875 116.88) (width 3) (layer "F.Cu") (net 26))
 (segment (start 123.415 122.965) (end 126.73 119.65) (width 3) (layer "F.Cu") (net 26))
 (segment (start 126.73 119.65) (end 126.73 116.8) (width 3) (layer "F.Cu") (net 26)))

